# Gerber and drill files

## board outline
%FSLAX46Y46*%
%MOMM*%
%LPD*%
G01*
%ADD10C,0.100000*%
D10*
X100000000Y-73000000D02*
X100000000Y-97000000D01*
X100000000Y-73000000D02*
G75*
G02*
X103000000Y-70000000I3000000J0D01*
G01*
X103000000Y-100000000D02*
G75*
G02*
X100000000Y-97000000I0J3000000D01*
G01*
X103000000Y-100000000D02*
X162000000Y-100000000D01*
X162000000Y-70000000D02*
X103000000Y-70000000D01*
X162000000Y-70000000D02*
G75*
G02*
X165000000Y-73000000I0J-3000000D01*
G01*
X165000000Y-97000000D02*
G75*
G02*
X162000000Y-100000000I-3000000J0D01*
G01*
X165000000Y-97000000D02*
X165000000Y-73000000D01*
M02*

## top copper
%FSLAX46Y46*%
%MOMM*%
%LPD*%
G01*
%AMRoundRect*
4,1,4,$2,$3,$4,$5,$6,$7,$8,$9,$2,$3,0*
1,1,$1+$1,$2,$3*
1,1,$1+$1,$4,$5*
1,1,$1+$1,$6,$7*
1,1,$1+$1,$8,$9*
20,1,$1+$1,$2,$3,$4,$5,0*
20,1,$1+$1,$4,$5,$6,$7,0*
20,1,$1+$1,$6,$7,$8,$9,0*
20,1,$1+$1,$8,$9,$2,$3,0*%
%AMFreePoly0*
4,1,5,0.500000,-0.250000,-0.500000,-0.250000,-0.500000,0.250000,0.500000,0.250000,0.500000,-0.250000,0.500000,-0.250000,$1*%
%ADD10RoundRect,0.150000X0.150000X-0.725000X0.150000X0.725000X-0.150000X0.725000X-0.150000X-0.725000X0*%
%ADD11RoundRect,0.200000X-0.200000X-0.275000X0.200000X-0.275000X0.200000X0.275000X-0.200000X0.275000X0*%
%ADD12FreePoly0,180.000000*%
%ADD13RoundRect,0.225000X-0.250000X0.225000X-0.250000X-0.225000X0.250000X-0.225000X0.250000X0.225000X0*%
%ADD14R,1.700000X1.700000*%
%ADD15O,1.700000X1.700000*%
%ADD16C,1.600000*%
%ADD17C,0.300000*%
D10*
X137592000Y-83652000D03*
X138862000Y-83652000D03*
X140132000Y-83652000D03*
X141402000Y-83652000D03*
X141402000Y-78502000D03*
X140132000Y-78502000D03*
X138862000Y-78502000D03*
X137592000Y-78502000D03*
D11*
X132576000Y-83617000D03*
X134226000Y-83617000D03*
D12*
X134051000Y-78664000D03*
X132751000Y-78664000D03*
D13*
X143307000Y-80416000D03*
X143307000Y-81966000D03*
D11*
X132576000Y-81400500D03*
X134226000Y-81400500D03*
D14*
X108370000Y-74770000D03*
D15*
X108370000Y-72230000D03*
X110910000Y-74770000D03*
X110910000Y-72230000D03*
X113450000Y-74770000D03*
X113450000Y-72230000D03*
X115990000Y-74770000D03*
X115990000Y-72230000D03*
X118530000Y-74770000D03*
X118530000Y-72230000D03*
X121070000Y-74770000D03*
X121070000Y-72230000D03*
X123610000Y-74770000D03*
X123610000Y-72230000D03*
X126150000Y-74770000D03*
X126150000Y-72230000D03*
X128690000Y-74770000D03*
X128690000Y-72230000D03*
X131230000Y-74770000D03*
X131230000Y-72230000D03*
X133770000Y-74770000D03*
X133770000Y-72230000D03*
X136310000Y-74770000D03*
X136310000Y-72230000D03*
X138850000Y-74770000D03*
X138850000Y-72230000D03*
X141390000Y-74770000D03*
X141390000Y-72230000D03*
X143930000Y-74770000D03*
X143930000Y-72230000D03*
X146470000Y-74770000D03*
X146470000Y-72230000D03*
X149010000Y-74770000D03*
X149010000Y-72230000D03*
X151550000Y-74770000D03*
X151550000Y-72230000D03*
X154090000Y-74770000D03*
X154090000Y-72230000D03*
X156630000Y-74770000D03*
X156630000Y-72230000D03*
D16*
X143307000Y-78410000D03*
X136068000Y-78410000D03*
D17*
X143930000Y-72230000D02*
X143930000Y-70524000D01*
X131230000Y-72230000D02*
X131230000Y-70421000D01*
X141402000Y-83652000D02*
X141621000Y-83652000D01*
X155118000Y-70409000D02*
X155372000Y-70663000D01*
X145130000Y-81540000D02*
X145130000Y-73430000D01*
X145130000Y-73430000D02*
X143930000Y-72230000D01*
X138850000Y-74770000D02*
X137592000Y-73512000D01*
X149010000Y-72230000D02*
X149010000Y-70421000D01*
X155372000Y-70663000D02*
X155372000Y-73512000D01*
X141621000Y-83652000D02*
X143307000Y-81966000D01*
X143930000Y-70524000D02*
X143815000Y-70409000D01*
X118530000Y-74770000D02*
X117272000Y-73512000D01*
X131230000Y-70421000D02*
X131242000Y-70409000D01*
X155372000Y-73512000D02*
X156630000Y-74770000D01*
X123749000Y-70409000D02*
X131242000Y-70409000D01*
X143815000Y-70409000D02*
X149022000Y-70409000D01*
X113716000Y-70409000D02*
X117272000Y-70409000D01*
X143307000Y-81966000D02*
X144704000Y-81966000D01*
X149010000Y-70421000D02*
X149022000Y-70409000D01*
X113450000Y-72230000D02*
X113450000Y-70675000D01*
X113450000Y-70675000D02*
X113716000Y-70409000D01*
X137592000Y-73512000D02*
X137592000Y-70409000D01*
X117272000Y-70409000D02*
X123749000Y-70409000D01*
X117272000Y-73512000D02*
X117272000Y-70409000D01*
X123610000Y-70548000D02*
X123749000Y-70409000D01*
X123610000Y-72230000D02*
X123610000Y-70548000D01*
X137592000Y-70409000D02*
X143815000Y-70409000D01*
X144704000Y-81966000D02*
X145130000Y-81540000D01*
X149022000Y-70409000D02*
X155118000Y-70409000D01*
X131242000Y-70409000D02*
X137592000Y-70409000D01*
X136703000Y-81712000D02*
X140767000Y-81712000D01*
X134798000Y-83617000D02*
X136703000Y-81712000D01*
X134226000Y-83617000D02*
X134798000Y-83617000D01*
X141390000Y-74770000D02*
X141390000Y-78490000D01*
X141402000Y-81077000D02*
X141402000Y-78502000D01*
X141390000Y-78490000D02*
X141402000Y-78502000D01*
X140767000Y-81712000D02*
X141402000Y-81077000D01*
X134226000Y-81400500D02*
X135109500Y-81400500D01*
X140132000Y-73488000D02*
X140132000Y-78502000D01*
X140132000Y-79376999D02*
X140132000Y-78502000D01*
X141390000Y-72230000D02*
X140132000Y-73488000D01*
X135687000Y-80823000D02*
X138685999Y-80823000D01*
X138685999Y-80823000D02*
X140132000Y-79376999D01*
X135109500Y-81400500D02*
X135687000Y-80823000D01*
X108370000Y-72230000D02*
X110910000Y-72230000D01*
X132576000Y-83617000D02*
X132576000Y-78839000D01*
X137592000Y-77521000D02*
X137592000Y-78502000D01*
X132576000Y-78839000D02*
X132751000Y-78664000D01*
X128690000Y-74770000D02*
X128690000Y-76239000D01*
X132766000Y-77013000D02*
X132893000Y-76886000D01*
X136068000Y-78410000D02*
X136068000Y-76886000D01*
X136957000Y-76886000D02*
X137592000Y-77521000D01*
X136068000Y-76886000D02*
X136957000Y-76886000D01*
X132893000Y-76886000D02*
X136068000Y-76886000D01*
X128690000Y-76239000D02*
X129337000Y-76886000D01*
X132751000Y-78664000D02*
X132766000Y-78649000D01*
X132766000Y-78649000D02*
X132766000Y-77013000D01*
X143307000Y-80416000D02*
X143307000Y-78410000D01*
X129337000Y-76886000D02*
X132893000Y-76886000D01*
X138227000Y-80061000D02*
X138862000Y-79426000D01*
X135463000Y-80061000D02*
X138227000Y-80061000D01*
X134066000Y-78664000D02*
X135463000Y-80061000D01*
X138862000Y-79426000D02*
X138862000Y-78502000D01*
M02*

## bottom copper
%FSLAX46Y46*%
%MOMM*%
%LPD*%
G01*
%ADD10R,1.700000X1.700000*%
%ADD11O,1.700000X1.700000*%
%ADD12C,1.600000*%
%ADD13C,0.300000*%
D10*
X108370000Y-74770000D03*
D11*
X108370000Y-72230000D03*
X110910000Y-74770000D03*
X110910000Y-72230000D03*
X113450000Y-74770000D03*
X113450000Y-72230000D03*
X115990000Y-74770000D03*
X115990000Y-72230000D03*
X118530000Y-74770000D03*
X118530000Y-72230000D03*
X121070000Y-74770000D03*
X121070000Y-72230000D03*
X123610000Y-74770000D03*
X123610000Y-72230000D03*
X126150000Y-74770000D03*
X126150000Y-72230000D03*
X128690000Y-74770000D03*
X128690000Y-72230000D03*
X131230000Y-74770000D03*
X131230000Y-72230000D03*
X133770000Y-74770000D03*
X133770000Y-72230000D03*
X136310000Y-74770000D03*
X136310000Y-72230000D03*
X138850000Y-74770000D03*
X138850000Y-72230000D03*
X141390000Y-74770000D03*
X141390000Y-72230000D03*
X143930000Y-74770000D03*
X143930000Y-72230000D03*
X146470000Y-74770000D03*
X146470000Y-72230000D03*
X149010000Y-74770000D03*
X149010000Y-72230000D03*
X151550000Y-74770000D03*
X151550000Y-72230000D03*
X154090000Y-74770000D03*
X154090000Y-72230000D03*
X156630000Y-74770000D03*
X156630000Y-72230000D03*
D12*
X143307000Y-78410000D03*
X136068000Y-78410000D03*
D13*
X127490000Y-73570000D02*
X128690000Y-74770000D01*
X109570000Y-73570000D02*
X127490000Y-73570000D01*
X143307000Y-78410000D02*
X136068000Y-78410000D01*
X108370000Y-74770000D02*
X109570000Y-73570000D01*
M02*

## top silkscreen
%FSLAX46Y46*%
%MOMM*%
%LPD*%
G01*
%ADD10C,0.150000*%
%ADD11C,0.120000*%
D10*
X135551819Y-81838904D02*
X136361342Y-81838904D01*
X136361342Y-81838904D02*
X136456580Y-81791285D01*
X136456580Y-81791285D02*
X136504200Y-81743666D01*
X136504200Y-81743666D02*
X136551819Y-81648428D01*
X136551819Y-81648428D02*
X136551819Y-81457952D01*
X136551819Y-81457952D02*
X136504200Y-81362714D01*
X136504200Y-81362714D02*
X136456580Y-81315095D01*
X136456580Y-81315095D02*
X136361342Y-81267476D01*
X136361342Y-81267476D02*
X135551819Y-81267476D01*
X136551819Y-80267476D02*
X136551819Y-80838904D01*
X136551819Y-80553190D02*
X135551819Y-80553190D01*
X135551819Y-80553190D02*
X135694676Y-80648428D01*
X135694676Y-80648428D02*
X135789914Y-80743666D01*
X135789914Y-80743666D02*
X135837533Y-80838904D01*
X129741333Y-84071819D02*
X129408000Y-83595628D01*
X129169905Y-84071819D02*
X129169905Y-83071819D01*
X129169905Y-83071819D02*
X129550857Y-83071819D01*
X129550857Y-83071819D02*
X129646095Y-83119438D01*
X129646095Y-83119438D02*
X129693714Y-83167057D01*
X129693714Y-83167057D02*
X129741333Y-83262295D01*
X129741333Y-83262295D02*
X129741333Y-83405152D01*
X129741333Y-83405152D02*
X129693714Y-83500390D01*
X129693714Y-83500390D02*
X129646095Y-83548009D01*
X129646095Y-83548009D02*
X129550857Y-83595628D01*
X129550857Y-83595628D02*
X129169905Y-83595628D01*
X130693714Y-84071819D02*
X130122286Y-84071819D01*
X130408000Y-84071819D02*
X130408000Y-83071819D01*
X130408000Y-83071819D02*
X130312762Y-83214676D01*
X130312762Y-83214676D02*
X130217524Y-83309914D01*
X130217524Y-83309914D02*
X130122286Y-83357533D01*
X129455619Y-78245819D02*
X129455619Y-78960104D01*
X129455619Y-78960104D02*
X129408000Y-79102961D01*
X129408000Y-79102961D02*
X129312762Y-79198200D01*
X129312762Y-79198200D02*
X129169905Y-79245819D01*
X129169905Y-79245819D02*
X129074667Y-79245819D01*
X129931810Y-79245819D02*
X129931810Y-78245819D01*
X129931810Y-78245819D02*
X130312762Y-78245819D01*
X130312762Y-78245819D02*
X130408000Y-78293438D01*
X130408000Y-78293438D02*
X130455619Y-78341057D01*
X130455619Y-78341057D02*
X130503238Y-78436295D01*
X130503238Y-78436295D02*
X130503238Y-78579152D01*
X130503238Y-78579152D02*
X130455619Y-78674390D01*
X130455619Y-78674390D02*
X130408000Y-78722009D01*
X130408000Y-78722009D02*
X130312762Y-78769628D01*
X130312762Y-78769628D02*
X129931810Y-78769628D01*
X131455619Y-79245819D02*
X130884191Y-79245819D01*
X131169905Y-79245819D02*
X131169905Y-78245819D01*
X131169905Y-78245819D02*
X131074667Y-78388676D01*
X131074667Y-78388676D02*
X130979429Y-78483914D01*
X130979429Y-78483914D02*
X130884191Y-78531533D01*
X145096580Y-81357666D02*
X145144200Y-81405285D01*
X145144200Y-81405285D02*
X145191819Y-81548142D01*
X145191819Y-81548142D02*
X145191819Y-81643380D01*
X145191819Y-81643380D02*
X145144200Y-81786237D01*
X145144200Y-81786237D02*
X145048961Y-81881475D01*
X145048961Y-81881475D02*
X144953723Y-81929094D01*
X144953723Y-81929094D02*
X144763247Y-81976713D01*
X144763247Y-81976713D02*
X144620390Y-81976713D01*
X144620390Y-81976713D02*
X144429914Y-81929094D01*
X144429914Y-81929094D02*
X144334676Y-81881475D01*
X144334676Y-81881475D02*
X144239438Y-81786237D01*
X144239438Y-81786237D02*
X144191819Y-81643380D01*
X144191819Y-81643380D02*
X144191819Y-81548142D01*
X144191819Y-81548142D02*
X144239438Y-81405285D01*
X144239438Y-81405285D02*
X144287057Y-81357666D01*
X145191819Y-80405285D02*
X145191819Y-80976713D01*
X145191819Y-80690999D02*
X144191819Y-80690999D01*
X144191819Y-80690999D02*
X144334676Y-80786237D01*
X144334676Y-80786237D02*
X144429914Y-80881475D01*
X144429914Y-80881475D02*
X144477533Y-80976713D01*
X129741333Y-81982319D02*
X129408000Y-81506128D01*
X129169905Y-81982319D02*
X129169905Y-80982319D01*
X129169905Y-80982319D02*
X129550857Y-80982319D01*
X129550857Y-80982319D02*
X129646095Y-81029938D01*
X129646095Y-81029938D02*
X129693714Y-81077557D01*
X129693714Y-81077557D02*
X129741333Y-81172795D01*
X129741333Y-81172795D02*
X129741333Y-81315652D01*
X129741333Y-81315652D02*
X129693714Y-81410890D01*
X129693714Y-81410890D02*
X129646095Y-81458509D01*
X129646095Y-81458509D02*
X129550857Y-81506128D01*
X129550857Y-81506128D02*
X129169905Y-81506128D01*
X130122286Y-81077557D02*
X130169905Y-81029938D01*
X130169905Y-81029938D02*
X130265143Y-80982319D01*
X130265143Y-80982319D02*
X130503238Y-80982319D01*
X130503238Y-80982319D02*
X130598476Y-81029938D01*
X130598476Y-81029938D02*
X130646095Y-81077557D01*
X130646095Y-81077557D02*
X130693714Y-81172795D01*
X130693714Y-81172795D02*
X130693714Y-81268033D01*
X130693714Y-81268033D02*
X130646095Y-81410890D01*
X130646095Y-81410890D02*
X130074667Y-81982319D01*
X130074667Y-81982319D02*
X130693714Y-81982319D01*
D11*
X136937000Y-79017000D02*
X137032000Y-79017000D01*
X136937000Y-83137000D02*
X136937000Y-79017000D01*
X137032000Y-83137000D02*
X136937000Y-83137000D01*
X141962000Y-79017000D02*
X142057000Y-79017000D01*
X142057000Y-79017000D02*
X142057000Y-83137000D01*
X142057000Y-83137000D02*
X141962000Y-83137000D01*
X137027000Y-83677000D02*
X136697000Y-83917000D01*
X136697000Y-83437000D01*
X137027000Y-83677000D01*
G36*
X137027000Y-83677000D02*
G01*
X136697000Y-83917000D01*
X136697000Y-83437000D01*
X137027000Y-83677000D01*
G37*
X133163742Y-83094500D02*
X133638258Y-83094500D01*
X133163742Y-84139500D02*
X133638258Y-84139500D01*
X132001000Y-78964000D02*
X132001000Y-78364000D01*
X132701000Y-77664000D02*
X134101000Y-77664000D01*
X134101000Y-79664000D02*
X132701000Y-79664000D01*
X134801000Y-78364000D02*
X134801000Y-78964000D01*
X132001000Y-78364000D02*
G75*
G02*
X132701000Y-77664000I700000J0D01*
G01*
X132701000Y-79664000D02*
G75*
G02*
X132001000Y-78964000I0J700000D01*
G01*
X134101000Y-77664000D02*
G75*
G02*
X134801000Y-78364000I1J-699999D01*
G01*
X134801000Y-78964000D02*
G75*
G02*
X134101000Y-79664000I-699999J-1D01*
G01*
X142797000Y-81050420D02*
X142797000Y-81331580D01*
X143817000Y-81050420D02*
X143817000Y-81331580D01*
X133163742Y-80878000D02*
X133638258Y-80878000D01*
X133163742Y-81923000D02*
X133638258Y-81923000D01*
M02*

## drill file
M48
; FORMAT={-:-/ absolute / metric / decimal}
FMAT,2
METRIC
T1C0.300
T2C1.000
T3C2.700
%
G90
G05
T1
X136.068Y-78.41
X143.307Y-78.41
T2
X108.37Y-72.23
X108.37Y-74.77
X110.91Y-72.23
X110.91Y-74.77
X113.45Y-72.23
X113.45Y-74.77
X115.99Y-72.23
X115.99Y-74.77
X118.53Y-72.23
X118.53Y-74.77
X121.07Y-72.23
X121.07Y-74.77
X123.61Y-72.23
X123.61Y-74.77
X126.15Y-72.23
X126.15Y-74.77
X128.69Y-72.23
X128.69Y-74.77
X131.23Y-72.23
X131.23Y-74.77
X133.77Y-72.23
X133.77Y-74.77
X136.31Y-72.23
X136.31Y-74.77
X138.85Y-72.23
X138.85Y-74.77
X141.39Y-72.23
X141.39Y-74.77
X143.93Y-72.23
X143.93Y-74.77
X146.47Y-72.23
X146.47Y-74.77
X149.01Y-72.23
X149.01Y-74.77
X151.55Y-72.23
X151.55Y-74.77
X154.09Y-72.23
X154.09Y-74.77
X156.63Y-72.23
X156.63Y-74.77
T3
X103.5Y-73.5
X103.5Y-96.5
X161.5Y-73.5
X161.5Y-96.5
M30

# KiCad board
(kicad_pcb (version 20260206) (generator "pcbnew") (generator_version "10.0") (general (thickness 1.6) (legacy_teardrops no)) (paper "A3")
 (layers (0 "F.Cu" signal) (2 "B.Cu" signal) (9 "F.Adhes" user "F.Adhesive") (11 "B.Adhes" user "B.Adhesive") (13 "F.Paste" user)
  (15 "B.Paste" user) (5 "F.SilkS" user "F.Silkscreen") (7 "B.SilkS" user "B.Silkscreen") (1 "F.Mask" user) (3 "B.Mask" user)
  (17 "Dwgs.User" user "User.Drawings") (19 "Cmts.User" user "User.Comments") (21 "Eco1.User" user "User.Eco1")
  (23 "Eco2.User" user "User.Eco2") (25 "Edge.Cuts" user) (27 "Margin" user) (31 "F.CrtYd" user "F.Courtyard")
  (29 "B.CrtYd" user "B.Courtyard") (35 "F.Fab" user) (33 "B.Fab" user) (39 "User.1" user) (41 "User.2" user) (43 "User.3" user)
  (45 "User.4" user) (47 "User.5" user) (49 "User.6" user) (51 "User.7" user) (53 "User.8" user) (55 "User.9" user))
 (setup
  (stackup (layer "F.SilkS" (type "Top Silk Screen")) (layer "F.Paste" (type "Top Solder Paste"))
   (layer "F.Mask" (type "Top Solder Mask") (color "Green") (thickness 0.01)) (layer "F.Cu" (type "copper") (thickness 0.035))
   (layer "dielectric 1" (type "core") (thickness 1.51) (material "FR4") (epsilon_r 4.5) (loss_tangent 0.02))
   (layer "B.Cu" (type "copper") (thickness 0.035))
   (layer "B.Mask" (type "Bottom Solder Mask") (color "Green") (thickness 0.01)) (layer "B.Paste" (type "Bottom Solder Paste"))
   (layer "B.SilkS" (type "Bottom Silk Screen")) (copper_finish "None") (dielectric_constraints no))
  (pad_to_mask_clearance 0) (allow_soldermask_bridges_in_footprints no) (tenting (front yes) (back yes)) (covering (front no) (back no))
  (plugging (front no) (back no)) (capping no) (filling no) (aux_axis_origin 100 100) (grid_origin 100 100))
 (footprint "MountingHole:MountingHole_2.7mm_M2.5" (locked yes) (layer "F.Cu") (at 161.5 73.5)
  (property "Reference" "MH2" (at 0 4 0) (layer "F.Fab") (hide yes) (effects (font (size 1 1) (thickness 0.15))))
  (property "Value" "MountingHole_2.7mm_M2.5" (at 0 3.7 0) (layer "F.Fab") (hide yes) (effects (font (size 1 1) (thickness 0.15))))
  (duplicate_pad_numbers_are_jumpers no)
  (pad "" np_thru_hole circle (at 0 0) (size 2.7 2.7) (drill 2.7) (layers "*.Cu" "*.Mask")))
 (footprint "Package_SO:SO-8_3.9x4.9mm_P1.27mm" (layer "F.Cu") (at 139.497 81.077 90)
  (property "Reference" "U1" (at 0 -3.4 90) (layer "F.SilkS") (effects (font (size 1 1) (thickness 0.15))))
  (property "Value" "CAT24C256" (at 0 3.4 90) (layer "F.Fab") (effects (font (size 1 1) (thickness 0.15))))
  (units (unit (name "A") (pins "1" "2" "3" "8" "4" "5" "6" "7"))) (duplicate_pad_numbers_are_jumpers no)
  (fp_line (start 2.06 -2.56) (end 2.06 -2.465) (stroke (width 0.12) (type solid)) (layer "F.SilkS"))
  (fp_line (start -2.06 -2.56) (end 2.06 -2.56) (stroke (width 0.12) (type solid)) (layer "F.SilkS"))
  (fp_line (start -2.06 -2.465) (end -2.06 -2.56) (stroke (width 0.12) (type solid)) (layer "F.SilkS"))
  (fp_line (start 2.06 2.465) (end 2.06 2.56) (stroke (width 0.12) (type solid)) (layer "F.SilkS"))
  (fp_line (start 2.06 2.56) (end -2.06 2.56) (stroke (width 0.12) (type solid)) (layer "F.SilkS"))
  (fp_line (start -2.06 2.56) (end -2.06 2.465) (stroke (width 0.12) (type solid)) (layer "F.SilkS"))
  (fp_poly (pts (xy -2.6 -2.47) (xy -2.84 -2.8) (xy -2.36 -2.8)) (stroke (width 0.12) (type solid)) (fill yes) (layer "F.SilkS"))
  (pad "1" smd roundrect (at -2.575 -1.905 90) (size 1.75 0.6) (layers "F.Cu" "F.Mask" "F.Paste") (roundrect_rratio 0.25)
   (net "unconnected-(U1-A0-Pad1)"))
  (pad "2" smd roundrect (at -2.575 -0.635 90) (size 1.75 0.6) (layers "F.Cu" "F.Mask" "F.Paste") (roundrect_rratio 0.25)
   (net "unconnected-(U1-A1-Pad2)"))
  (pad "3" smd roundrect (at -2.575 0.635 90) (size 1.75 0.6) (layers "F.Cu" "F.Mask" "F.Paste") (roundrect_rratio 0.25)
   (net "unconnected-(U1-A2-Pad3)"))
  (pad "4" smd roundrect (at -2.575 1.905 90) (size 1.75 0.6) (layers "F.Cu" "F.Mask" "F.Paste") (roundrect_rratio 0.25) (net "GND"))
  (pad "5" smd roundrect (at 2.575 1.905 90) (size 1.75 0.6) (layers "F.Cu" "F.Mask" "F.Paste") (roundrect_rratio 0.25) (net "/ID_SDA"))
  (pad "6" smd roundrect (at 2.575 0.635 90) (size 1.75 0.6) (layers "F.Cu" "F.Mask" "F.Paste") (roundrect_rratio 0.25) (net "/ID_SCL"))
  (pad "7" smd roundrect (at 2.575 -0.635 90) (size 1.75 0.6) (layers "F.Cu" "F.Mask" "F.Paste") (roundrect_rratio 0.25) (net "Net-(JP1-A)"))
  (pad "8" smd roundrect (at 2.575 -1.905 90) (size 1.75 0.6) (layers "F.Cu" "F.Mask" "F.Paste") (roundrect_rratio 0.25) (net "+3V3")))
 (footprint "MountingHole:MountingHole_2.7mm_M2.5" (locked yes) (layer "F.Cu") (at 103.5 96.5)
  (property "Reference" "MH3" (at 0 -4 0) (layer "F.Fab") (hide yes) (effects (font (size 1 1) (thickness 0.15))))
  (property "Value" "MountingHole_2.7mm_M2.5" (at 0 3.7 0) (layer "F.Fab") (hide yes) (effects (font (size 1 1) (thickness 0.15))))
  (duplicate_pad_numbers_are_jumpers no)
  (pad "" np_thru_hole circle (at 0 0) (size 2.7 2.7) (drill 2.7) (layers "*.Cu" "*.Mask")))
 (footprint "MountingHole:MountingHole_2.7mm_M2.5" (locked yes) (layer "F.Cu") (at 103.5 73.5)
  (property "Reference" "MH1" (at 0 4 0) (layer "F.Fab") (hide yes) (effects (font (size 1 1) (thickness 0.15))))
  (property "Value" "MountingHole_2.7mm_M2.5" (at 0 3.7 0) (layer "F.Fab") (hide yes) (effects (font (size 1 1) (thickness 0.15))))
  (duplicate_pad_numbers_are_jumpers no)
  (pad "" np_thru_hole circle (at 0 0) (size 2.7 2.7) (drill 2.7) (layers "*.Cu" "*.Mask")))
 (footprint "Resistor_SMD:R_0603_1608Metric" (layer "F.Cu") (at 133.401 83.617)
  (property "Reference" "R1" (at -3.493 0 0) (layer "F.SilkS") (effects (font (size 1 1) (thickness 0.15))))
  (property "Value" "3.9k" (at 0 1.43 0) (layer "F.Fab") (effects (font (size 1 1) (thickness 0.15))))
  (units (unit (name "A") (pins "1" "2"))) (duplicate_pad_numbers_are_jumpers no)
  (fp_line (start -0.237258 -0.5225) (end 0.237258 -0.5225) (stroke (width 0.12) (type solid)) (layer "F.SilkS"))
  (fp_line (start -0.237258 0.5225) (end 0.237258 0.5225) (stroke (width 0.12) (type solid)) (layer "F.SilkS"))
  (pad "1" smd roundrect (at -0.825 0) (size 0.8 0.95) (layers "F.Cu" "F.Mask" "F.Paste") (roundrect_rratio 0.25) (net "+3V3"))
  (pad "2" smd roundrect (at 0.825 0) (size 0.8 0.95) (layers "F.Cu" "F.Mask" "F.Paste") (roundrect_rratio 0.25) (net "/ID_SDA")))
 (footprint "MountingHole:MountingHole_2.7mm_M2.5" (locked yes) (layer "F.Cu") (at 161.5 96.5)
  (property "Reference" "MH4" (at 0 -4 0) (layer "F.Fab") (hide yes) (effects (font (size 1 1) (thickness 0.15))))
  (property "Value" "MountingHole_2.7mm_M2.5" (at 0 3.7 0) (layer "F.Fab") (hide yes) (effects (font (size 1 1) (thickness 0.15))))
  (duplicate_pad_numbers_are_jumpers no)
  (pad "" np_thru_hole circle (at 0 0) (size 2.7 2.7) (drill 2.7) (layers "*.Cu" "*.Mask")))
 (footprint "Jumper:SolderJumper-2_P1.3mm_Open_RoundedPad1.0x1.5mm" (layer "F.Cu") (at 133.401 78.664 180)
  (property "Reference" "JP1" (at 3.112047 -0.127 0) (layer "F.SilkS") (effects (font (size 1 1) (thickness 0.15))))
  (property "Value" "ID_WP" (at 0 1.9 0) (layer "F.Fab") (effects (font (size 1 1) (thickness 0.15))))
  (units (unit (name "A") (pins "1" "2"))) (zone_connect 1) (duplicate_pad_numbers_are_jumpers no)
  (fp_line (start 1.4 -0.3) (end 1.4 0.3) (stroke (width 0.12) (type solid)) (layer "F.SilkS"))
  (fp_line (start 0.7 1) (end -0.7 1) (stroke (width 0.12) (type solid)) (layer "F.SilkS"))
  (fp_line (start -0.7 -1) (end 0.7 -1) (stroke (width 0.12) (type solid)) (layer "F.SilkS"))
  (fp_line (start -1.4 0.3) (end -1.4 -0.3) (stroke (width 0.12) (type solid)) (layer "F.SilkS"))
  (fp_arc (start 1.4 0.3) (mid 1.194975 0.794975) (end 0.7 1) (stroke (width 0.12) (type solid)) (layer "F.SilkS"))
  (fp_arc (start 0.7 -1) (mid 1.194975 -0.794975) (end 1.4 -0.3) (stroke (width 0.12) (type solid)) (layer "F.SilkS"))
  (fp_arc (start -0.7 1) (mid -1.194975 0.794975) (end -1.4 0.3) (stroke (width 0.12) (type solid)) (layer "F.SilkS"))
  (fp_arc (start -1.4 -0.3) (mid -1.194975 -0.794975) (end -0.7 -1) (stroke (width 0.12) (type solid)) (layer "F.SilkS"))
  (pad "1" smd custom (at -0.65 0 180) (size 1 0.5) (layers "F.Cu" "F.Mask") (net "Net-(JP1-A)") (zone_connect 2) (thermal_bridge_angle 45)
   (options (clearance outline) (anchor rect)) (primitives))
  (pad "2" smd custom (at 0.65 0 180) (size 1 0.5) (layers "F.Cu" "F.Mask") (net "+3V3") (zone_connect 2) (thermal_bridge_angle 45)
   (options (clearance outline) (anchor rect)) (primitives)))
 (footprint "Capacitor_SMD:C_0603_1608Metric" (layer "F.Cu") (at 143.307 81.191 -90)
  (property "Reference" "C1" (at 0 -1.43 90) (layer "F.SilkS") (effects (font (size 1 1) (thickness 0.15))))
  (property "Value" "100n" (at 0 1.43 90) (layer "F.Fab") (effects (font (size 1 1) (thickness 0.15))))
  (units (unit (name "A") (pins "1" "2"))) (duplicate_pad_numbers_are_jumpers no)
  (fp_line (start -0.14058 0.51) (end 0.14058 0.51) (stroke (width 0.12) (type solid)) (layer "F.SilkS"))
  (fp_line (start -0.14058 -0.51) (end 0.14058 -0.51) (stroke (width 0.12) (type solid)) (layer "F.SilkS"))
  (pad "1" smd roundrect (at -0.775 0 270) (size 0.9 0.95) (layers "F.Cu" "F.Mask" "F.Paste") (roundrect_rratio 0.25) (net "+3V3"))
  (pad "2" smd roundrect (at 0.775 0 270) (size 0.9 0.95) (layers "F.Cu" "F.Mask" "F.Paste") (roundrect_rratio 0.25) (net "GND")))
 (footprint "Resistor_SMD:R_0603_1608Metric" (layer "F.Cu") (at 133.401 81.4005)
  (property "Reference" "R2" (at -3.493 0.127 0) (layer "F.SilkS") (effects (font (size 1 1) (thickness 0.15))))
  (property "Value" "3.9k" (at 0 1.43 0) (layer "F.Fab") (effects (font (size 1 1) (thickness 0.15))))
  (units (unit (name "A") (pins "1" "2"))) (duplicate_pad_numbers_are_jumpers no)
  (fp_line (start -0.237258 -0.5225) (end 0.237258 -0.5225) (stroke (width 0.12) (type solid)) (layer "F.SilkS"))
  (fp_line (start -0.237258 0.5225) (end 0.237258 0.5225) (stroke (width 0.12) (type solid)) (layer "F.SilkS"))
  (pad "1" smd roundrect (at -0.825 0) (size 0.8 0.95) (layers "F.Cu" "F.Mask" "F.Paste") (roundrect_rratio 0.25) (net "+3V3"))
  (pad "2" smd roundrect (at 0.825 0) (size 0.8 0.95) (layers "F.Cu" "F.Mask" "F.Paste") (roundrect_rratio 0.25) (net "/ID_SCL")))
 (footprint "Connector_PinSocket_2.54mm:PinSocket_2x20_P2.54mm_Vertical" (layer "B.Cu") (at 108.37 74.77 -90)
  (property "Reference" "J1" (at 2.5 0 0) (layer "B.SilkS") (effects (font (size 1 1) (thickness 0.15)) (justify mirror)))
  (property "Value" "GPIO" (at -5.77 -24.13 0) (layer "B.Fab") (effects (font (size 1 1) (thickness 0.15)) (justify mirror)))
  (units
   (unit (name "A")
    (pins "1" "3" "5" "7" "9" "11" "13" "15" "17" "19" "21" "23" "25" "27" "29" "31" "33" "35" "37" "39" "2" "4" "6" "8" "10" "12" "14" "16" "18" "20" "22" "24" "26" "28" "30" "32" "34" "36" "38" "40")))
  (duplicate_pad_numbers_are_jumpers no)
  (pad "1" thru_hole rect (at 0 0 270) (size 1.7 1.7) (drill 1) (layers "*.Cu" "*.Mask") (remove_unused_layers no) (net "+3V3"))
  (pad "2" thru_hole oval (at -2.54 0 270) (size 1.7 1.7) (drill 1) (layers "*.Cu" "*.Mask") (remove_unused_layers no) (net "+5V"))
  (pad "3" thru_hole oval (at 0 -2.54 270) (size 1.7 1.7) (drill 1) (layers "*.Cu" "*.Mask") (remove_unused_layers no)
   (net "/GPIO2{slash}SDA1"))
  (pad "4" thru_hole oval (at -2.54 -2.54 270) (size 1.7 1.7) (drill 1) (layers "*.Cu" "*.Mask") (remove_unused_layers no) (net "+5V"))
  (pad "5" thru_hole oval (at 0 -5.08 270) (size 1.7 1.7) (drill 1) (layers "*.Cu" "*.Mask") (remove_unused_layers no)
   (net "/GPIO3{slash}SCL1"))
  (pad "6" thru_hole oval (at -2.54 -5.08 270) (size 1.7 1.7) (drill 1) (layers "*.Cu" "*.Mask") (remove_unused_layers no) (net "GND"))
  (pad "7" thru_hole oval (at 0 -7.62 270) (size 1.7 1.7) (drill 1) (layers "*.Cu" "*.Mask") (remove_unused_layers no)
   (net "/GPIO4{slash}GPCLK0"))
  (pad "8" thru_hole oval (at -2.54 -7.62 270) (size 1.7 1.7) (drill 1) (layers "*.Cu" "*.Mask") (remove_unused_layers no)
   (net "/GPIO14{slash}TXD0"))
  (pad "9" thru_hole oval (at 0 -10.16 270) (size 1.7 1.7) (drill 1) (layers "*.Cu" "*.Mask") (remove_unused_layers no) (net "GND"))
  (pad "10" thru_hole oval (at -2.54 -10.16 270) (size 1.7 1.7) (drill 1) (layers "*.Cu" "*.Mask") (remove_unused_layers no)
   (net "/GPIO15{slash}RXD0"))
  (pad "11" thru_hole oval (at 0 -12.7 270) (size 1.7 1.7) (drill 1) (layers "*.Cu" "*.Mask") (remove_unused_layers no) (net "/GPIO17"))
  (pad "12" thru_hole oval (at -2.54 -12.7 270) (size 1.7 1.7) (drill 1) (layers "*.Cu" "*.Mask") (remove_unused_layers no)
   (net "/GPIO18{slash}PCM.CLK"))
  (pad "13" thru_hole oval (at 0 -15.24 270) (size 1.7 1.7) (drill 1) (layers "*.Cu" "*.Mask") (remove_unused_layers no) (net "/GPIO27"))
  (pad "14" thru_hole oval (at -2.54 -15.24 270) (size 1.7 1.7) (drill 1) (layers "*.Cu" "*.Mask") (remove_unused_layers no) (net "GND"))
  (pad "15" thru_hole oval (at 0 -17.78 270) (size 1.7 1.7) (drill 1) (layers "*.Cu" "*.Mask") (remove_unused_layers no) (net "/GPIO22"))
  (pad "16" thru_hole oval (at -2.54 -17.78 270) (size 1.7 1.7) (drill 1) (layers "*.Cu" "*.Mask") (remove_unused_layers no) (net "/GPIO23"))
  (pad "17" thru_hole oval (at 0 -20.32 270) (size 1.7 1.7) (drill 1) (layers "*.Cu" "*.Mask") (remove_unused_layers no) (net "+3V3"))
  (pad "18" thru_hole oval (at -2.54 -20.32 270) (size 1.7 1.7) (drill 1) (layers "*.Cu" "*.Mask") (remove_unused_layers no) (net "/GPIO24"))
  (pad "19" thru_hole oval (at 0 -22.86 270) (size 1.7 1.7) (drill 1) (layers "*.Cu" "*.Mask") (remove_unused_layers no)
   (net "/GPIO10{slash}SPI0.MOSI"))
  (pad "20" thru_hole oval (at -2.54 -22.86 270) (size 1.7 1.7) (drill 1) (layers "*.Cu" "*.Mask") (remove_unused_layers no) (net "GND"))
  (pad "21" thru_hole oval (at 0 -25.4 270) (size 1.7 1.7) (drill 1) (layers "*.Cu" "*.Mask") (remove_unused_layers no)
   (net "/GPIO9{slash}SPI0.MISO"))
  (pad "22" thru_hole oval (at -2.54 -25.4 270) (size 1.7 1.7) (drill 1) (layers "*.Cu" "*.Mask") (remove_unused_layers no) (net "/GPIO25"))
  (pad "23" thru_hole oval (at 0 -27.94 270) (size 1.7 1.7) (drill 1) (layers "*.Cu" "*.Mask") (remove_unused_layers no)
   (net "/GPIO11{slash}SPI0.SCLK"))
  (pad "24" thru_hole oval (at -2.54 -27.94 270) (size 1.7 1.7) (drill 1) (layers "*.Cu" "*.Mask") (remove_unused_layers no)
   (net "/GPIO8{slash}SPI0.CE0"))
  (pad "25" thru_hole oval (at 0 -30.48 270) (size 1.7 1.7) (drill 1) (layers "*.Cu" "*.Mask") (remove_unused_layers no) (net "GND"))
  (pad "26" thru_hole oval (at -2.54 -30.48 270) (size 1.7 1.7) (drill 1) (layers "*.Cu" "*.Mask") (remove_unused_layers no)
   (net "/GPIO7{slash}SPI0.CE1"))
  (pad "27" thru_hole oval (at 0 -33.02 270) (size 1.7 1.7) (drill 1) (layers "*.Cu" "*.Mask") (remove_unused_layers no) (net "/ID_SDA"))
  (pad "28" thru_hole oval (at -2.54 -33.02 270) (size 1.7 1.7) (drill 1) (layers "*.Cu" "*.Mask") (remove_unused_layers no) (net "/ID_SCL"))
  (pad "29" thru_hole oval (at 0 -35.56 270) (size 1.7 1.7) (drill 1) (layers "*.Cu" "*.Mask") (remove_unused_layers no) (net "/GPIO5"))
  (pad "30" thru_hole oval (at -2.54 -35.56 270) (size 1.7 1.7) (drill 1) (layers "*.Cu" "*.Mask") (remove_unused_layers no) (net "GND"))
  (pad "31" thru_hole oval (at 0 -38.1 270) (size 1.7 1.7) (drill 1) (layers "*.Cu" "*.Mask") (remove_unused_layers no) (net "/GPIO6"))
  (pad "32" thru_hole oval (at -2.54 -38.1 270) (size 1.7 1.7) (drill 1) (layers "*.Cu" "*.Mask") (remove_unused_layers no)
   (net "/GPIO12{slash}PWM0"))
  (pad "33" thru_hole oval (at 0 -40.64 270) (size 1.7 1.7) (drill 1) (layers "*.Cu" "*.Mask") (remove_unused_layers no)
   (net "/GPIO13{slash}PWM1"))
  (pad "34" thru_hole oval (at -2.54 -40.64 270) (size 1.7 1.7) (drill 1) (layers "*.Cu" "*.Mask") (remove_unused_layers no) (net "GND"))
  (pad "35" thru_hole oval (at 0 -43.18 270) (size 1.7 1.7) (drill 1) (layers "*.Cu" "*.Mask") (remove_unused_layers no)
   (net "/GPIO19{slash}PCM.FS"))
  (pad "36" thru_hole oval (at -2.54 -43.18 270) (size 1.7 1.7) (drill 1) (layers "*.Cu" "*.Mask") (remove_unused_layers no) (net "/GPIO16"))
  (pad "37" thru_hole oval (at 0 -45.72 270) (size 1.7 1.7) (drill 1) (layers "*.Cu" "*.Mask") (remove_unused_layers no) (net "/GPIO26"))
  (pad "38" thru_hole oval (at -2.54 -45.72 270) (size 1.7 1.7) (drill 1) (layers "*.Cu" "*.Mask") (remove_unused_layers no)
   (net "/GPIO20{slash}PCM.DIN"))
  (pad "39" thru_hole oval (at 0 -48.26 270) (size 1.7 1.7) (drill 1) (layers "*.Cu" "*.Mask") (remove_unused_layers no) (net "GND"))
  (pad "40" thru_hole oval (at -2.54 -48.26 270) (size 1.7 1.7) (drill 1) (layers "*.Cu" "*.Mask") (remove_unused_layers no)
   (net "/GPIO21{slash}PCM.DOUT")))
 (gr_line (start 100 73) (end 100 97) (stroke (width 0.1) (type solid)) (layer "Edge.Cuts"))
 (gr_arc (start 100 73) (mid 100.87868 70.87868) (end 103 70) (stroke (width 0.1) (type solid)) (layer "Edge.Cuts"))
 (gr_arc (start 103 100) (mid 100.87868 99.12132) (end 100 97) (stroke (width 0.1) (type solid)) (layer "Edge.Cuts"))
 (gr_line (start 103 100) (end 162 100) (stroke (width 0.1) (type solid)) (layer "Edge.Cuts"))
 (gr_line (start 162 70) (end 103 70) (stroke (width 0.1) (type solid)) (layer "Edge.Cuts"))
 (gr_arc (start 162 70) (mid 164.12132 70.87868) (end 165 73) (stroke (width 0.1) (type solid)) (layer "Edge.Cuts"))
 (gr_arc (start 165 97) (mid 164.12132 99.12132) (end 162 100) (stroke (width 0.1) (type solid)) (layer "Edge.Cuts"))
 (gr_line (start 165 97) (end 165 73) (stroke (width 0.1) (type solid)) (layer "Edge.Cuts"))
 (segment (start 143.93 72.23) (end 143.93 70.524) (width 0.3) (layer "F.Cu") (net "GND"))
 (segment (start 131.23 72.23) (end 131.23 70.421) (width 0.3) (layer "F.Cu") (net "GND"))
 (segment (start 141.402 83.652) (end 141.621 83.652) (width 0.3) (layer "F.Cu") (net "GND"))
 (segment (start 155.118 70.409) (end 155.372 70.663) (width 0.3) (layer "F.Cu") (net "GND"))
 (segment (start 145.13 81.54) (end 145.13 73.43) (width 0.3) (layer "F.Cu") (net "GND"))
 (segment (start 145.13 73.43) (end 143.93 72.23) (width 0.3) (layer "F.Cu") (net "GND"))
 (segment (start 138.85 74.77) (end 137.592 73.512) (width 0.3) (layer "F.Cu") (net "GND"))
 (segment (start 149.01 72.23) (end 149.01 70.421) (width 0.3) (layer "F.Cu") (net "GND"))
 (segment (start 155.372 70.663) (end 155.372 73.512) (width 0.3) (layer "F.Cu") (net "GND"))
 (segment (start 141.621 83.652) (end 143.307 81.966) (width 0.3) (layer "F.Cu") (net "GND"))
 (segment (start 143.93 70.524) (end 143.815 70.409) (width 0.3) (layer "F.Cu") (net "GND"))
 (segment (start 118.53 74.77) (end 117.272 73.512) (width 0.3) (layer "F.Cu") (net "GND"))
 (segment (start 131.23 70.421) (end 131.242 70.409) (width 0.3) (layer "F.Cu") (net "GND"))
 (segment (start 155.372 73.512) (end 156.63 74.77) (width 0.3) (layer "F.Cu") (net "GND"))
 (segment (start 123.749 70.409) (end 131.242 70.409) (width 0.3) (layer "F.Cu") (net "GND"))
 (segment (start 143.815 70.409) (end 149.022 70.409) (width 0.3) (layer "F.Cu") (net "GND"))
 (segment (start 113.716 70.409) (end 117.272 70.409) (width 0.3) (layer "F.Cu") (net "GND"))
 (segment (start 143.307 81.966) (end 144.704 81.966) (width 0.3) (layer "F.Cu") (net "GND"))
 (segment (start 149.01 70.421) (end 149.022 70.409) (width 0.3) (layer "F.Cu") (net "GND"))
 (segment (start 113.45 72.23) (end 113.45 70.675) (width 0.3) (layer "F.Cu") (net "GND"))
 (segment (start 113.45 70.675) (end 113.716 70.409) (width 0.3) (layer "F.Cu") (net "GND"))
 (segment (start 137.592 73.512) (end 137.592 70.409) (width 0.3) (layer "F.Cu") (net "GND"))
 (segment (start 117.272 70.409) (end 123.749 70.409) (width 0.3) (layer "F.Cu") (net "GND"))
 (segment (start 117.272 73.512) (end 117.272 70.409) (width 0.3) (layer "F.Cu") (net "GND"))
 (segment (start 123.61 70.548) (end 123.749 70.409) (width 0.3) (layer "F.Cu") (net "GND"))
 (segment (start 123.61 72.23) (end 123.61 70.548) (width 0.3) (layer "F.Cu") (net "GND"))
 (segment (start 137.592 70.409) (end 143.815 70.409) (width 0.3) (layer "F.Cu") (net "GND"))
 (segment (start 144.704 81.966) (end 145.13 81.54) (width 0.3) (layer "F.Cu") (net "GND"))
 (segment (start 149.022 70.409) (end 155.118 70.409) (width 0.3) (layer "F.Cu") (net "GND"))
 (segment (start 131.242 70.409) (end 137.592 70.409) (width 0.3) (layer "F.Cu") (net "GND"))
 (segment (start 136.703 81.712) (end 140.767 81.712) (width 0.3) (layer "F.Cu") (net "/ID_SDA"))
 (segment (start 134.798 83.617) (end 136.703 81.712) (width 0.3) (layer "F.Cu") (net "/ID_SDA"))
 (segment (start 134.226 83.617) (end 134.798 83.617) (width 0.3) (layer "F.Cu") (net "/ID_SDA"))
 (segment (start 141.39 74.77) (end 141.39 78.49) (width 0.3) (layer "F.Cu") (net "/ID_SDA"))
 (segment (start 141.402 81.077) (end 141.402 78.502) (width 0.3) (layer "F.Cu") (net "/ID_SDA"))
 (segment (start 141.39 78.49) (end 141.402 78.502) (width 0.3) (layer "F.Cu") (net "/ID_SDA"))
 (segment (start 140.767 81.712) (end 141.402 81.077) (width 0.3) (layer "F.Cu") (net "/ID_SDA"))
 (segment (start 134.226 81.4005) (end 135.1095 81.4005) (width 0.3) (layer "F.Cu") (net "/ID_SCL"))
 (segment (start 140.132 73.488) (end 140.132 78.502) (width 0.3) (layer "F.Cu") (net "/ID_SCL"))
 (segment (start 140.132 79.376999) (end 140.132 78.502) (width 0.3) (layer "F.Cu") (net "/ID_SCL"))
 (segment (start 141.39 72.23) (end 140.132 73.488) (width 0.3) (layer "F.Cu") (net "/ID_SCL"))
 (segment (start 135.687 80.823) (end 138.685999 80.823) (width 0.3) (layer "F.Cu") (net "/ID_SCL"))
 (segment (start 138.685999 80.823) (end 140.132 79.376999) (width 0.3) (layer "F.Cu") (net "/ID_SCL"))
 (segment (start 135.1095 81.4005) (end 135.687 80.823) (width 0.3) (layer "F.Cu") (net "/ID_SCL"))
 (segment (start 108.37 72.23) (end 110.91 72.23) (width 0.3) (layer "F.Cu") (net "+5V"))
 (segment (start 132.576 83.617) (end 132.576 78.839) (width 0.3) (layer "F.Cu") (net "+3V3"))
 (segment (start 137.592 77.521) (end 137.592 78.502) (width 0.3) (layer "F.Cu") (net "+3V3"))
 (segment (start 132.576 78.839) (end 132.751 78.664) (width 0.3) (layer "F.Cu") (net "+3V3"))
 (segment (start 128.69 74.77) (end 128.69 76.239) (width 0.3) (layer "F.Cu") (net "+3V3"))
 (segment (start 132.766 77.013) (end 132.893 76.886) (width 0.3) (layer "F.Cu") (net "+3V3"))
 (segment (start 136.068 78.41) (end 136.068 76.886) (width 0.3) (layer "F.Cu") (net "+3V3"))
 (segment (start 136.957 76.886) (end 137.592 77.521) (width 0.3) (layer "F.Cu") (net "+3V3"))
 (segment (start 136.068 76.886) (end 136.957 76.886) (width 0.3) (layer "F.Cu") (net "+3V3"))
 (segment (start 132.893 76.886) (end 136.068 76.886) (width 0.3) (layer "F.Cu") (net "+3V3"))
 (segment (start 128.69 76.239) (end 129.337 76.886) (width 0.3) (layer "F.Cu") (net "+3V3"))
 (segment (start 132.751 78.664) (end 132.766 78.649) (width 0.3) (layer "F.Cu") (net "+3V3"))
 (segment (start 132.766 78.649) (end 132.766 77.013) (width 0.3) (layer "F.Cu") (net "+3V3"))
 (segment (start 143.307 80.416) (end 143.307 78.41) (width 0.3) (layer "F.Cu") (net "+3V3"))
 (segment (start 129.337 76.886) (end 132.893 76.886) (width 0.3) (layer "F.Cu") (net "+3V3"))
 (via (at 143.307 78.41) (size 1.6) (drill 0.3) (layers "F.Cu" "B.Cu") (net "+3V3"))
 (via (at 136.068 78.41) (size 1.6) (drill 0.3) (layers "F.Cu" "B.Cu") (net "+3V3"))
 (segment (start 127.49 73.57) (end 128.69 74.77) (width 0.3) (layer "B.Cu") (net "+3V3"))
 (segment (start 109.57 73.57) (end 127.49 73.57) (width 0.3) (layer "B.Cu") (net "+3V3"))
 (segment (start 143.307 78.41) (end 136.068 78.41) (width 0.3) (layer "B.Cu") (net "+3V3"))
 (segment (start 108.37 74.77) (end 109.57 73.57) (width 0.3) (layer "B.Cu") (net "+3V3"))
 (segment (start 138.227 80.061) (end 138.862 79.426) (width 0.3) (layer "F.Cu") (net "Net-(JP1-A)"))
 (segment (start 135.463 80.061) (end 138.227 80.061) (width 0.3) (layer "F.Cu") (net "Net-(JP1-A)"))
 (segment (start 134.066 78.664) (end 135.463 80.061) (width 0.3) (layer "F.Cu") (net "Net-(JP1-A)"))
 (segment (start 138.862 79.426) (end 138.862 78.502) (width 0.3) (layer "F.Cu") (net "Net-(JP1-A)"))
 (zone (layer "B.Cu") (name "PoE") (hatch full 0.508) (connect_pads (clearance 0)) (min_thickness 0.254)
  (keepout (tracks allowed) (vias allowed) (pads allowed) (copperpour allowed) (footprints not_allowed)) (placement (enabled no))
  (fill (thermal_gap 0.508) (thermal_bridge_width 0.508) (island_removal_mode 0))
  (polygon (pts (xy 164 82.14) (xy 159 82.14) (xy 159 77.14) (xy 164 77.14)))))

